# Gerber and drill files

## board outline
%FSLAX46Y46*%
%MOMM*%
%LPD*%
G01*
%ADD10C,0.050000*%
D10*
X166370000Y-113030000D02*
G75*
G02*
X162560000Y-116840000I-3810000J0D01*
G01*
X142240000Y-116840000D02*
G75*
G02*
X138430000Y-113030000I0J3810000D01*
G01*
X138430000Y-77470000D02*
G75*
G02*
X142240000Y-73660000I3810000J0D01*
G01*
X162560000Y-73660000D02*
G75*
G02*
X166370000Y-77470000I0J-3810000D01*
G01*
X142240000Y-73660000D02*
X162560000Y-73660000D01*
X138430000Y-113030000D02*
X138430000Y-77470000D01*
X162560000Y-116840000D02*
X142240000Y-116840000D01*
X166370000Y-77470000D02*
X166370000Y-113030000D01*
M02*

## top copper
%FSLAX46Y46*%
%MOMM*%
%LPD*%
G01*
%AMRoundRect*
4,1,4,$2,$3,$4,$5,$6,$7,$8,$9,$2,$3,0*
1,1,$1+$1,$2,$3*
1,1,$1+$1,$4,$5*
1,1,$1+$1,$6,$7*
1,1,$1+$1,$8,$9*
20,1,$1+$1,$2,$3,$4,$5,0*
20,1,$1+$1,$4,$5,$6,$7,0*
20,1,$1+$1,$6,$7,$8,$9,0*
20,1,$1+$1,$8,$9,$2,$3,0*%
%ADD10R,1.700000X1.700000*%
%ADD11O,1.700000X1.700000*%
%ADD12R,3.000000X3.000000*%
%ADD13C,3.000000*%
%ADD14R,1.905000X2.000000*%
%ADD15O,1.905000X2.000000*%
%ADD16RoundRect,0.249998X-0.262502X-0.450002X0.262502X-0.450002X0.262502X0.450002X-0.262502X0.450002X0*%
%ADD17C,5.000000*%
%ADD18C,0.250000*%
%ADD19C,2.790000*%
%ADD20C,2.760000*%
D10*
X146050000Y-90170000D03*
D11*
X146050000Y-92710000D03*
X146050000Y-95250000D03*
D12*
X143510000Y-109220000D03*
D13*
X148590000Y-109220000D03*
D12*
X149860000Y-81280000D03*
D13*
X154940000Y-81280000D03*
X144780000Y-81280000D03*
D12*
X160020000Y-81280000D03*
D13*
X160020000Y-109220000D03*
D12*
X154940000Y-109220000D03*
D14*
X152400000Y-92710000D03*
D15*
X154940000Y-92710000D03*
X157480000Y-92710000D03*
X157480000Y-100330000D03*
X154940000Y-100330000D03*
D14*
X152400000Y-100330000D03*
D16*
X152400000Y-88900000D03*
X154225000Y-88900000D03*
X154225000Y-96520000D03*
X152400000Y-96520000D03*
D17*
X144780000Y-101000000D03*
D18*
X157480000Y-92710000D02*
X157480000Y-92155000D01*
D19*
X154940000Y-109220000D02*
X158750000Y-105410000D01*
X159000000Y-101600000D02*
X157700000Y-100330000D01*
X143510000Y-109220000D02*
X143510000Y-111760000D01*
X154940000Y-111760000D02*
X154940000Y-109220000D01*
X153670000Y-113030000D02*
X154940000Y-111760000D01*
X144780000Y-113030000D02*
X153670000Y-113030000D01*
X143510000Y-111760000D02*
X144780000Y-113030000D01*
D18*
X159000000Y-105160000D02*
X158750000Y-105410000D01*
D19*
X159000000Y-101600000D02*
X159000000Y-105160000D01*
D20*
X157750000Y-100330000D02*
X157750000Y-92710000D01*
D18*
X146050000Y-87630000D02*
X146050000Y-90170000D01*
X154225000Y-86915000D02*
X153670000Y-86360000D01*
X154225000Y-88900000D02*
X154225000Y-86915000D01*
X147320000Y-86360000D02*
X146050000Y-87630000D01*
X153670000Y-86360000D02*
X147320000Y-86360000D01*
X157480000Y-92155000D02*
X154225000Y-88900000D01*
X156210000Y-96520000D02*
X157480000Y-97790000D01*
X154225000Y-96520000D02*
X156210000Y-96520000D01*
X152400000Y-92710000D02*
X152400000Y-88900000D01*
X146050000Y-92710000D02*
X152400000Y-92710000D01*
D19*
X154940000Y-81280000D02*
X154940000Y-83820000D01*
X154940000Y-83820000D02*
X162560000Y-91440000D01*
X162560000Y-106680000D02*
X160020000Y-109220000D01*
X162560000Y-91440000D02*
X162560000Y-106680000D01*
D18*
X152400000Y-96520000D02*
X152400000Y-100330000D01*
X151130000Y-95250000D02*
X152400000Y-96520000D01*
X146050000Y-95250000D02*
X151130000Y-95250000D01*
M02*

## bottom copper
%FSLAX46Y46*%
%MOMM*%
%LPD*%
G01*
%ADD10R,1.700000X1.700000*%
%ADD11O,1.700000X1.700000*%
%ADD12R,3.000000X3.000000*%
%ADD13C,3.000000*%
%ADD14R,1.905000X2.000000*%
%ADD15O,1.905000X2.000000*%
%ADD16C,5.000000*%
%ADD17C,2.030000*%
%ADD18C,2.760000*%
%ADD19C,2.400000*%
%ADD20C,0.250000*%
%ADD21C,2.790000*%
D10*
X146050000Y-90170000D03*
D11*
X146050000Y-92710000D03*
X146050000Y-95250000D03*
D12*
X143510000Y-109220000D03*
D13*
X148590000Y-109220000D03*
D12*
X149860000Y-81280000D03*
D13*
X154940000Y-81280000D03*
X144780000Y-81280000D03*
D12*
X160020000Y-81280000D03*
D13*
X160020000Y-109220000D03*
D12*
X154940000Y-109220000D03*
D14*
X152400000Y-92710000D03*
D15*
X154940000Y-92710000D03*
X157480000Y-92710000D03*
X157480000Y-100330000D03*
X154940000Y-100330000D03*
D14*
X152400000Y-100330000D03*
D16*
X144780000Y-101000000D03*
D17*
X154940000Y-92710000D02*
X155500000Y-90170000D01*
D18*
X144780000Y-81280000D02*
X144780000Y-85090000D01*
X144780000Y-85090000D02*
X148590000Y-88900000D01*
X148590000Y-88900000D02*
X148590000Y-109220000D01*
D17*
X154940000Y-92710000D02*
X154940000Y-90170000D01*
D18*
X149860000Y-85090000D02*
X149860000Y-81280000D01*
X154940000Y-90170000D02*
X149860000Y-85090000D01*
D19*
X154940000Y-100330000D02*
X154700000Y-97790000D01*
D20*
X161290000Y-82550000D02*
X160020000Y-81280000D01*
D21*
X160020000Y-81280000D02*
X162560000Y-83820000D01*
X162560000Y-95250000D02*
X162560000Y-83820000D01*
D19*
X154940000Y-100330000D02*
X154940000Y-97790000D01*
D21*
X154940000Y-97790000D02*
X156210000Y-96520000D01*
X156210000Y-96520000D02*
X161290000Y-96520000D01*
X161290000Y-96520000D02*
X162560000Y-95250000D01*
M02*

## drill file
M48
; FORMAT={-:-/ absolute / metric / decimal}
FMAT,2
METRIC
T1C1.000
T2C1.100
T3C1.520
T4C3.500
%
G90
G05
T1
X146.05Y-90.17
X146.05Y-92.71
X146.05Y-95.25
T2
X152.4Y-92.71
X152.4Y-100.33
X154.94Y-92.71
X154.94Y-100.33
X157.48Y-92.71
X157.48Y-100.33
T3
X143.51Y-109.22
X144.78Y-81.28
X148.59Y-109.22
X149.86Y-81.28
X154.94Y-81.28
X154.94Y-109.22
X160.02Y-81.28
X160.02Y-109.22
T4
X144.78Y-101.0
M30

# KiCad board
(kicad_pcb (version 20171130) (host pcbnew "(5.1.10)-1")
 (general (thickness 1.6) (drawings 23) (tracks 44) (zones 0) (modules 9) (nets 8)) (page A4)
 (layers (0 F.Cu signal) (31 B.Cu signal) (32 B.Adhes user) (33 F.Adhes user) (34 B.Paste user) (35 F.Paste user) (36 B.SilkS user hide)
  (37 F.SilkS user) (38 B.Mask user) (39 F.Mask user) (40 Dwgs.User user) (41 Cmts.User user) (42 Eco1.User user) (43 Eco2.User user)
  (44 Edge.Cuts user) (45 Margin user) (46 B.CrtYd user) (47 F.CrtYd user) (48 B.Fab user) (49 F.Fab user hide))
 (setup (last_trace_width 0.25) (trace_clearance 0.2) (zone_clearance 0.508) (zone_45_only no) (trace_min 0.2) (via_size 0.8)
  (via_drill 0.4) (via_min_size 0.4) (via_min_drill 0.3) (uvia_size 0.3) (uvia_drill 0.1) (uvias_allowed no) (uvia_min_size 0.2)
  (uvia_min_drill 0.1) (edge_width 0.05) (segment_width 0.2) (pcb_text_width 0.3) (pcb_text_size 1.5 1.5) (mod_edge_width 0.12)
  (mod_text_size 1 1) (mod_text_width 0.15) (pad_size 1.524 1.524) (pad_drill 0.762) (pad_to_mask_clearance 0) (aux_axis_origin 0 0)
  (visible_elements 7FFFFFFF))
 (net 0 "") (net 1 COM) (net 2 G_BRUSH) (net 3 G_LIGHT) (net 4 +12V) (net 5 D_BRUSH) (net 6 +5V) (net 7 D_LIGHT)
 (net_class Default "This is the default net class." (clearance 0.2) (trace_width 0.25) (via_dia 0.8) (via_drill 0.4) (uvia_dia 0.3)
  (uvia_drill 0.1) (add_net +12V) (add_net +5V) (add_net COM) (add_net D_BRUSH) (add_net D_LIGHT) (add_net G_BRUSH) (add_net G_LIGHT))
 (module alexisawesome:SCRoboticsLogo (layer B.Cu) (at 156.21 86.36 180)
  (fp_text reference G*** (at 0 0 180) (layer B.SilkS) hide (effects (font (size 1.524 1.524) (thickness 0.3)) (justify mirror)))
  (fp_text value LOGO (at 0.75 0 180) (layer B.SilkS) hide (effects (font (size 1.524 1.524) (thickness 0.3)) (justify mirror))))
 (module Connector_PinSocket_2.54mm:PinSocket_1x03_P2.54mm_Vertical (layer F.Cu) (at 146.05 90.17)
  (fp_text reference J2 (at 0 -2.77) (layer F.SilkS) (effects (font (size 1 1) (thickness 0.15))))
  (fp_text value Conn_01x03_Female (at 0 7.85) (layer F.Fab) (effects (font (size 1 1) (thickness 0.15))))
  (pad 1 thru_hole rect (at 0 0) (size 1.7 1.7) (drill 1) (layers *.Cu *.Mask) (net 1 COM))
  (pad 2 thru_hole oval (at 0 2.54) (size 1.7 1.7) (drill 1) (layers *.Cu *.Mask) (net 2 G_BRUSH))
  (pad 3 thru_hole oval (at 0 5.08) (size 1.7 1.7) (drill 1) (layers *.Cu *.Mask) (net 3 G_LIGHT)))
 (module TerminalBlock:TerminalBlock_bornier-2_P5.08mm (layer F.Cu) (at 143.51 109.22)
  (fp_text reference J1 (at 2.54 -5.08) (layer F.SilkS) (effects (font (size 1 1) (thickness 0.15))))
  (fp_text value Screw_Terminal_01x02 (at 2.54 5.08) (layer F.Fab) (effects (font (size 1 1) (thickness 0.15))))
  (pad 1 thru_hole rect (at 0 0) (size 3 3) (drill 1.52) (layers *.Cu *.Mask) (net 1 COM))
  (pad 2 thru_hole circle (at 5.08 0) (size 3 3) (drill 1.52) (layers *.Cu *.Mask) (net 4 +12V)))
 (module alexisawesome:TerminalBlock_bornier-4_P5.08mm (layer F.Cu) (at 144.78 81.28)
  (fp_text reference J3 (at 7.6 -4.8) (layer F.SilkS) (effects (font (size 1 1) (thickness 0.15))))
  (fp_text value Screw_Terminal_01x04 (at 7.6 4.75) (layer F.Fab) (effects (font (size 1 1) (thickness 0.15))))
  (pad 2 thru_hole rect (at 5.08 0) (size 3 3) (drill 1.52) (layers *.Cu *.Mask) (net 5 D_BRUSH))
  (pad 3 thru_hole circle (at 10.16 0) (size 3 3) (drill 1.52) (layers *.Cu *.Mask) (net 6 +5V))
  (pad 1 thru_hole circle (at 0 0) (size 3 3) (drill 1.52) (layers *.Cu *.Mask) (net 4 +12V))
  (pad 4 thru_hole rect (at 15.24 0) (size 3 3) (drill 1.52) (layers *.Cu *.Mask) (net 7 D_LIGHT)))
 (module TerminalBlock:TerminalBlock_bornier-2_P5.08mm (layer F.Cu) (at 154.94 109.22)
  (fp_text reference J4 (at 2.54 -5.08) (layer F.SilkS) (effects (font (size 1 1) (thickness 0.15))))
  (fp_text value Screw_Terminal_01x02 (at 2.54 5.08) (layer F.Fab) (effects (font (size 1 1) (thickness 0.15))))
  (pad 2 thru_hole circle (at 5.08 0) (size 3 3) (drill 1.52) (layers *.Cu *.Mask) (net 6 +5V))
  (pad 1 thru_hole rect (at 0 0) (size 3 3) (drill 1.52) (layers *.Cu *.Mask) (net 1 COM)))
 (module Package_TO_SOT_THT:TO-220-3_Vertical (layer F.Cu) (at 152.4 92.71)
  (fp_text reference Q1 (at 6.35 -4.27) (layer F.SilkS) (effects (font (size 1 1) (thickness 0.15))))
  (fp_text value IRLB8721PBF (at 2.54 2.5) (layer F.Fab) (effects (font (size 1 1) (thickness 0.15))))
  (pad 1 thru_hole rect (at 0 0) (size 1.905 2) (drill 1.1) (layers *.Cu *.Mask) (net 2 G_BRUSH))
  (pad 2 thru_hole oval (at 2.54 0) (size 1.905 2) (drill 1.1) (layers *.Cu *.Mask) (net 5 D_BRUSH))
  (pad 3 thru_hole oval (at 5.08 0) (size 1.905 2) (drill 1.1) (layers *.Cu *.Mask) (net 1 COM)))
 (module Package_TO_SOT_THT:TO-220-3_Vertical (layer F.Cu) (at 152.4 100.33)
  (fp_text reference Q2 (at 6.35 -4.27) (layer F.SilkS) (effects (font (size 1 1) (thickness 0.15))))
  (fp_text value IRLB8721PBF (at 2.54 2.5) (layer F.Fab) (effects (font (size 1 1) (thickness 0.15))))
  (pad 3 thru_hole oval (at 5.08 0) (size 1.905 2) (drill 1.1) (layers *.Cu *.Mask) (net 1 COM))
  (pad 2 thru_hole oval (at 2.54 0) (size 1.905 2) (drill 1.1) (layers *.Cu *.Mask) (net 7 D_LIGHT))
  (pad 1 thru_hole rect (at 0 0) (size 1.905 2) (drill 1.1) (layers *.Cu *.Mask) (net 3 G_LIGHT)))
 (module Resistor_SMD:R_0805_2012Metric (layer F.Cu) (at 153.3125 88.9)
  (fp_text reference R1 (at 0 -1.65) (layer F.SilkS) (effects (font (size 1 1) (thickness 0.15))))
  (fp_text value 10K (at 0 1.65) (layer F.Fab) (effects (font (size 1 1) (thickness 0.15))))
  (pad 1 smd roundrect (at -0.9125 0) (size 1.025 1.4) (layers F.Cu F.Paste F.Mask) (roundrect_rratio 0.2439004878048781) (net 2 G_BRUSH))
  (pad 2 smd roundrect (at 0.9125 0) (size 1.025 1.4) (layers F.Cu F.Paste F.Mask) (roundrect_rratio 0.2439004878048781) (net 1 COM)))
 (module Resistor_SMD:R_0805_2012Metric (layer F.Cu) (at 153.3125 96.52)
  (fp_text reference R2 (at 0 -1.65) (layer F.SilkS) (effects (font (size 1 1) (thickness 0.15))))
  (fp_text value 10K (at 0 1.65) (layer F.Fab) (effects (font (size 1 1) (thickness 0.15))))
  (pad 2 smd roundrect (at 0.9125 0) (size 1.025 1.4) (layers F.Cu F.Paste F.Mask) (roundrect_rratio 0.2439004878048781) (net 1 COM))
  (pad 1 smd roundrect (at -0.9125 0) (size 1.025 1.4) (layers F.Cu F.Paste F.Mask) (roundrect_rratio 0.2439004878048781) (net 3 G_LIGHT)))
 (gr_arc (start 162.56 113.03) (end 162.56 116.84) (angle -90) (layer Edge.Cuts) (width 0.05))
 (gr_arc (start 142.24 113.03) (end 138.43 113.03) (angle -90) (layer Edge.Cuts) (width 0.05))
 (gr_arc (start 142.24 77.47) (end 142.24 73.66) (angle -90) (layer Edge.Cuts) (width 0.05))
 (gr_arc (start 162.56 77.47) (end 166.37 77.47) (angle -90) (layer Edge.Cuts) (width 0.05))
 (gr_line (start 142.24 73.66) (end 162.56 73.66) (layer Edge.Cuts) (width 0.05))
 (gr_line (start 138.43 113.03) (end 138.43 77.47) (layer Edge.Cuts) (width 0.05))
 (gr_line (start 162.56 116.84) (end 142.24 116.84) (layer Edge.Cuts) (width 0.05))
 (gr_line (start 166.37 77.47) (end 166.37 113.03) (layer Edge.Cuts) (width 0.05))
 (via (at 144.78 101) (size 5) (drill 3.5) (layers F.Cu B.Cu) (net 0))
 (segment (start 154.94 92.71) (end 155.5 90.17) (width 2.03) (layer B.Cu) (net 5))
 (segment (start 144.78 81.28) (end 144.78 85.09) (width 2.76) (layer B.Cu) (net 4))
 (segment (start 144.78 85.09) (end 148.59 88.9) (width 2.76) (layer B.Cu) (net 4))
 (segment (start 148.59 88.9) (end 148.59 109.22) (width 2.76) (layer B.Cu) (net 4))
 (segment (start 154.94 92.71) (end 154.94 90.17) (width 2.03) (layer B.Cu) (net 5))
 (segment (start 149.86 85.09) (end 149.86 81.28) (width 2.76) (layer B.Cu) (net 5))
 (segment (start 154.94 90.17) (end 149.86 85.09) (width 2.76) (layer B.Cu) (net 5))
 (segment (start 157.48 92.71) (end 157.48 92.155) (width 0.25) (layer F.Cu) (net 1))
 (segment (start 154.94 109.22) (end 158.75 105.41) (width 2.79) (layer F.Cu) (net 1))
 (segment (start 159 101.6) (end 157.7 100.33) (width 2.79) (layer F.Cu) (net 1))
 (segment (start 143.51 109.22) (end 143.51 111.76) (width 2.79) (layer F.Cu) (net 1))
 (segment (start 154.94 111.76) (end 154.94 109.22) (width 2.79) (layer F.Cu) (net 1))
 (segment (start 153.67 113.03) (end 154.94 111.76) (width 2.79) (layer F.Cu) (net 1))
 (segment (start 144.78 113.03) (end 153.67 113.03) (width 2.79) (layer F.Cu) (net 1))
 (segment (start 143.51 111.76) (end 144.78 113.03) (width 2.79) (layer F.Cu) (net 1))
 (segment (start 159 105.16) (end 158.75 105.41) (width 0.25) (layer F.Cu) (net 1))
 (segment (start 159 101.6) (end 159 105.16) (width 2.79) (layer F.Cu) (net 1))
 (segment (start 157.75 100.33) (end 157.75 92.71) (width 2.76) (layer F.Cu) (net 1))
 (segment (start 146.05 87.63) (end 146.05 90.17) (width 0.25) (layer F.Cu) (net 1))
 (segment (start 154.225 86.915) (end 153.67 86.36) (width 0.25) (layer F.Cu) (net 1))
 (segment (start 154.225 88.9) (end 154.225 86.915) (width 0.25) (layer F.Cu) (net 1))
 (segment (start 147.32 86.36) (end 146.05 87.63) (width 0.25) (layer F.Cu) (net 1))
 (segment (start 153.67 86.36) (end 147.32 86.36) (width 0.25) (layer F.Cu) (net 1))
 (segment (start 157.48 92.155) (end 154.225 88.9) (width 0.25) (layer F.Cu) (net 1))
 (segment (start 156.21 96.52) (end 157.48 97.79) (width 0.25) (layer F.Cu) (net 1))
 (segment (start 154.225 96.52) (end 156.21 96.52) (width 0.25) (layer F.Cu) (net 1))
 (segment (start 152.4 92.71) (end 152.4 88.9) (width 0.25) (layer F.Cu) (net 2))
 (segment (start 146.05 92.71) (end 152.4 92.71) (width 0.25) (layer F.Cu) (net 2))
 (segment (start 154.94 100.33) (end 154.7 97.79) (width 2.4) (layer B.Cu) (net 7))
 (segment (start 161.29 82.55) (end 160.02 81.28) (width 0.25) (layer B.Cu) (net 7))
 (segment (start 160.02 81.28) (end 162.56 83.82) (width 2.79) (layer B.Cu) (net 7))
 (segment (start 162.56 95.25) (end 162.56 83.82) (width 2.79) (layer B.Cu) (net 7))
 (segment (start 154.94 100.33) (end 154.94 97.79) (width 2.4) (layer B.Cu) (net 7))
 (segment (start 154.94 97.79) (end 156.21 96.52) (width 2.79) (layer B.Cu) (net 7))
 (segment (start 156.21 96.52) (end 161.29 96.52) (width 2.79) (layer B.Cu) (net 7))
 (segment (start 161.29 96.52) (end 162.56 95.25) (width 2.79) (layer B.Cu) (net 7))
 (segment (start 154.94 81.28) (end 154.94 83.82) (width 2.79) (layer F.Cu) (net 6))
 (segment (start 154.94 83.82) (end 162.56 91.44) (width 2.79) (layer F.Cu) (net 6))
 (segment (start 162.56 106.68) (end 160.02 109.22) (width 2.79) (layer F.Cu) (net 6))
 (segment (start 162.56 91.44) (end 162.56 106.68) (width 2.79) (layer F.Cu) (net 6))
 (segment (start 152.4 96.52) (end 152.4 100.33) (width 0.25) (layer F.Cu) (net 3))
 (segment (start 151.13 95.25) (end 152.4 96.52) (width 0.25) (layer F.Cu) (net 3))
 (segment (start 146.05 95.25) (end 151.13 95.25) (width 0.25) (layer F.Cu) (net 3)))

